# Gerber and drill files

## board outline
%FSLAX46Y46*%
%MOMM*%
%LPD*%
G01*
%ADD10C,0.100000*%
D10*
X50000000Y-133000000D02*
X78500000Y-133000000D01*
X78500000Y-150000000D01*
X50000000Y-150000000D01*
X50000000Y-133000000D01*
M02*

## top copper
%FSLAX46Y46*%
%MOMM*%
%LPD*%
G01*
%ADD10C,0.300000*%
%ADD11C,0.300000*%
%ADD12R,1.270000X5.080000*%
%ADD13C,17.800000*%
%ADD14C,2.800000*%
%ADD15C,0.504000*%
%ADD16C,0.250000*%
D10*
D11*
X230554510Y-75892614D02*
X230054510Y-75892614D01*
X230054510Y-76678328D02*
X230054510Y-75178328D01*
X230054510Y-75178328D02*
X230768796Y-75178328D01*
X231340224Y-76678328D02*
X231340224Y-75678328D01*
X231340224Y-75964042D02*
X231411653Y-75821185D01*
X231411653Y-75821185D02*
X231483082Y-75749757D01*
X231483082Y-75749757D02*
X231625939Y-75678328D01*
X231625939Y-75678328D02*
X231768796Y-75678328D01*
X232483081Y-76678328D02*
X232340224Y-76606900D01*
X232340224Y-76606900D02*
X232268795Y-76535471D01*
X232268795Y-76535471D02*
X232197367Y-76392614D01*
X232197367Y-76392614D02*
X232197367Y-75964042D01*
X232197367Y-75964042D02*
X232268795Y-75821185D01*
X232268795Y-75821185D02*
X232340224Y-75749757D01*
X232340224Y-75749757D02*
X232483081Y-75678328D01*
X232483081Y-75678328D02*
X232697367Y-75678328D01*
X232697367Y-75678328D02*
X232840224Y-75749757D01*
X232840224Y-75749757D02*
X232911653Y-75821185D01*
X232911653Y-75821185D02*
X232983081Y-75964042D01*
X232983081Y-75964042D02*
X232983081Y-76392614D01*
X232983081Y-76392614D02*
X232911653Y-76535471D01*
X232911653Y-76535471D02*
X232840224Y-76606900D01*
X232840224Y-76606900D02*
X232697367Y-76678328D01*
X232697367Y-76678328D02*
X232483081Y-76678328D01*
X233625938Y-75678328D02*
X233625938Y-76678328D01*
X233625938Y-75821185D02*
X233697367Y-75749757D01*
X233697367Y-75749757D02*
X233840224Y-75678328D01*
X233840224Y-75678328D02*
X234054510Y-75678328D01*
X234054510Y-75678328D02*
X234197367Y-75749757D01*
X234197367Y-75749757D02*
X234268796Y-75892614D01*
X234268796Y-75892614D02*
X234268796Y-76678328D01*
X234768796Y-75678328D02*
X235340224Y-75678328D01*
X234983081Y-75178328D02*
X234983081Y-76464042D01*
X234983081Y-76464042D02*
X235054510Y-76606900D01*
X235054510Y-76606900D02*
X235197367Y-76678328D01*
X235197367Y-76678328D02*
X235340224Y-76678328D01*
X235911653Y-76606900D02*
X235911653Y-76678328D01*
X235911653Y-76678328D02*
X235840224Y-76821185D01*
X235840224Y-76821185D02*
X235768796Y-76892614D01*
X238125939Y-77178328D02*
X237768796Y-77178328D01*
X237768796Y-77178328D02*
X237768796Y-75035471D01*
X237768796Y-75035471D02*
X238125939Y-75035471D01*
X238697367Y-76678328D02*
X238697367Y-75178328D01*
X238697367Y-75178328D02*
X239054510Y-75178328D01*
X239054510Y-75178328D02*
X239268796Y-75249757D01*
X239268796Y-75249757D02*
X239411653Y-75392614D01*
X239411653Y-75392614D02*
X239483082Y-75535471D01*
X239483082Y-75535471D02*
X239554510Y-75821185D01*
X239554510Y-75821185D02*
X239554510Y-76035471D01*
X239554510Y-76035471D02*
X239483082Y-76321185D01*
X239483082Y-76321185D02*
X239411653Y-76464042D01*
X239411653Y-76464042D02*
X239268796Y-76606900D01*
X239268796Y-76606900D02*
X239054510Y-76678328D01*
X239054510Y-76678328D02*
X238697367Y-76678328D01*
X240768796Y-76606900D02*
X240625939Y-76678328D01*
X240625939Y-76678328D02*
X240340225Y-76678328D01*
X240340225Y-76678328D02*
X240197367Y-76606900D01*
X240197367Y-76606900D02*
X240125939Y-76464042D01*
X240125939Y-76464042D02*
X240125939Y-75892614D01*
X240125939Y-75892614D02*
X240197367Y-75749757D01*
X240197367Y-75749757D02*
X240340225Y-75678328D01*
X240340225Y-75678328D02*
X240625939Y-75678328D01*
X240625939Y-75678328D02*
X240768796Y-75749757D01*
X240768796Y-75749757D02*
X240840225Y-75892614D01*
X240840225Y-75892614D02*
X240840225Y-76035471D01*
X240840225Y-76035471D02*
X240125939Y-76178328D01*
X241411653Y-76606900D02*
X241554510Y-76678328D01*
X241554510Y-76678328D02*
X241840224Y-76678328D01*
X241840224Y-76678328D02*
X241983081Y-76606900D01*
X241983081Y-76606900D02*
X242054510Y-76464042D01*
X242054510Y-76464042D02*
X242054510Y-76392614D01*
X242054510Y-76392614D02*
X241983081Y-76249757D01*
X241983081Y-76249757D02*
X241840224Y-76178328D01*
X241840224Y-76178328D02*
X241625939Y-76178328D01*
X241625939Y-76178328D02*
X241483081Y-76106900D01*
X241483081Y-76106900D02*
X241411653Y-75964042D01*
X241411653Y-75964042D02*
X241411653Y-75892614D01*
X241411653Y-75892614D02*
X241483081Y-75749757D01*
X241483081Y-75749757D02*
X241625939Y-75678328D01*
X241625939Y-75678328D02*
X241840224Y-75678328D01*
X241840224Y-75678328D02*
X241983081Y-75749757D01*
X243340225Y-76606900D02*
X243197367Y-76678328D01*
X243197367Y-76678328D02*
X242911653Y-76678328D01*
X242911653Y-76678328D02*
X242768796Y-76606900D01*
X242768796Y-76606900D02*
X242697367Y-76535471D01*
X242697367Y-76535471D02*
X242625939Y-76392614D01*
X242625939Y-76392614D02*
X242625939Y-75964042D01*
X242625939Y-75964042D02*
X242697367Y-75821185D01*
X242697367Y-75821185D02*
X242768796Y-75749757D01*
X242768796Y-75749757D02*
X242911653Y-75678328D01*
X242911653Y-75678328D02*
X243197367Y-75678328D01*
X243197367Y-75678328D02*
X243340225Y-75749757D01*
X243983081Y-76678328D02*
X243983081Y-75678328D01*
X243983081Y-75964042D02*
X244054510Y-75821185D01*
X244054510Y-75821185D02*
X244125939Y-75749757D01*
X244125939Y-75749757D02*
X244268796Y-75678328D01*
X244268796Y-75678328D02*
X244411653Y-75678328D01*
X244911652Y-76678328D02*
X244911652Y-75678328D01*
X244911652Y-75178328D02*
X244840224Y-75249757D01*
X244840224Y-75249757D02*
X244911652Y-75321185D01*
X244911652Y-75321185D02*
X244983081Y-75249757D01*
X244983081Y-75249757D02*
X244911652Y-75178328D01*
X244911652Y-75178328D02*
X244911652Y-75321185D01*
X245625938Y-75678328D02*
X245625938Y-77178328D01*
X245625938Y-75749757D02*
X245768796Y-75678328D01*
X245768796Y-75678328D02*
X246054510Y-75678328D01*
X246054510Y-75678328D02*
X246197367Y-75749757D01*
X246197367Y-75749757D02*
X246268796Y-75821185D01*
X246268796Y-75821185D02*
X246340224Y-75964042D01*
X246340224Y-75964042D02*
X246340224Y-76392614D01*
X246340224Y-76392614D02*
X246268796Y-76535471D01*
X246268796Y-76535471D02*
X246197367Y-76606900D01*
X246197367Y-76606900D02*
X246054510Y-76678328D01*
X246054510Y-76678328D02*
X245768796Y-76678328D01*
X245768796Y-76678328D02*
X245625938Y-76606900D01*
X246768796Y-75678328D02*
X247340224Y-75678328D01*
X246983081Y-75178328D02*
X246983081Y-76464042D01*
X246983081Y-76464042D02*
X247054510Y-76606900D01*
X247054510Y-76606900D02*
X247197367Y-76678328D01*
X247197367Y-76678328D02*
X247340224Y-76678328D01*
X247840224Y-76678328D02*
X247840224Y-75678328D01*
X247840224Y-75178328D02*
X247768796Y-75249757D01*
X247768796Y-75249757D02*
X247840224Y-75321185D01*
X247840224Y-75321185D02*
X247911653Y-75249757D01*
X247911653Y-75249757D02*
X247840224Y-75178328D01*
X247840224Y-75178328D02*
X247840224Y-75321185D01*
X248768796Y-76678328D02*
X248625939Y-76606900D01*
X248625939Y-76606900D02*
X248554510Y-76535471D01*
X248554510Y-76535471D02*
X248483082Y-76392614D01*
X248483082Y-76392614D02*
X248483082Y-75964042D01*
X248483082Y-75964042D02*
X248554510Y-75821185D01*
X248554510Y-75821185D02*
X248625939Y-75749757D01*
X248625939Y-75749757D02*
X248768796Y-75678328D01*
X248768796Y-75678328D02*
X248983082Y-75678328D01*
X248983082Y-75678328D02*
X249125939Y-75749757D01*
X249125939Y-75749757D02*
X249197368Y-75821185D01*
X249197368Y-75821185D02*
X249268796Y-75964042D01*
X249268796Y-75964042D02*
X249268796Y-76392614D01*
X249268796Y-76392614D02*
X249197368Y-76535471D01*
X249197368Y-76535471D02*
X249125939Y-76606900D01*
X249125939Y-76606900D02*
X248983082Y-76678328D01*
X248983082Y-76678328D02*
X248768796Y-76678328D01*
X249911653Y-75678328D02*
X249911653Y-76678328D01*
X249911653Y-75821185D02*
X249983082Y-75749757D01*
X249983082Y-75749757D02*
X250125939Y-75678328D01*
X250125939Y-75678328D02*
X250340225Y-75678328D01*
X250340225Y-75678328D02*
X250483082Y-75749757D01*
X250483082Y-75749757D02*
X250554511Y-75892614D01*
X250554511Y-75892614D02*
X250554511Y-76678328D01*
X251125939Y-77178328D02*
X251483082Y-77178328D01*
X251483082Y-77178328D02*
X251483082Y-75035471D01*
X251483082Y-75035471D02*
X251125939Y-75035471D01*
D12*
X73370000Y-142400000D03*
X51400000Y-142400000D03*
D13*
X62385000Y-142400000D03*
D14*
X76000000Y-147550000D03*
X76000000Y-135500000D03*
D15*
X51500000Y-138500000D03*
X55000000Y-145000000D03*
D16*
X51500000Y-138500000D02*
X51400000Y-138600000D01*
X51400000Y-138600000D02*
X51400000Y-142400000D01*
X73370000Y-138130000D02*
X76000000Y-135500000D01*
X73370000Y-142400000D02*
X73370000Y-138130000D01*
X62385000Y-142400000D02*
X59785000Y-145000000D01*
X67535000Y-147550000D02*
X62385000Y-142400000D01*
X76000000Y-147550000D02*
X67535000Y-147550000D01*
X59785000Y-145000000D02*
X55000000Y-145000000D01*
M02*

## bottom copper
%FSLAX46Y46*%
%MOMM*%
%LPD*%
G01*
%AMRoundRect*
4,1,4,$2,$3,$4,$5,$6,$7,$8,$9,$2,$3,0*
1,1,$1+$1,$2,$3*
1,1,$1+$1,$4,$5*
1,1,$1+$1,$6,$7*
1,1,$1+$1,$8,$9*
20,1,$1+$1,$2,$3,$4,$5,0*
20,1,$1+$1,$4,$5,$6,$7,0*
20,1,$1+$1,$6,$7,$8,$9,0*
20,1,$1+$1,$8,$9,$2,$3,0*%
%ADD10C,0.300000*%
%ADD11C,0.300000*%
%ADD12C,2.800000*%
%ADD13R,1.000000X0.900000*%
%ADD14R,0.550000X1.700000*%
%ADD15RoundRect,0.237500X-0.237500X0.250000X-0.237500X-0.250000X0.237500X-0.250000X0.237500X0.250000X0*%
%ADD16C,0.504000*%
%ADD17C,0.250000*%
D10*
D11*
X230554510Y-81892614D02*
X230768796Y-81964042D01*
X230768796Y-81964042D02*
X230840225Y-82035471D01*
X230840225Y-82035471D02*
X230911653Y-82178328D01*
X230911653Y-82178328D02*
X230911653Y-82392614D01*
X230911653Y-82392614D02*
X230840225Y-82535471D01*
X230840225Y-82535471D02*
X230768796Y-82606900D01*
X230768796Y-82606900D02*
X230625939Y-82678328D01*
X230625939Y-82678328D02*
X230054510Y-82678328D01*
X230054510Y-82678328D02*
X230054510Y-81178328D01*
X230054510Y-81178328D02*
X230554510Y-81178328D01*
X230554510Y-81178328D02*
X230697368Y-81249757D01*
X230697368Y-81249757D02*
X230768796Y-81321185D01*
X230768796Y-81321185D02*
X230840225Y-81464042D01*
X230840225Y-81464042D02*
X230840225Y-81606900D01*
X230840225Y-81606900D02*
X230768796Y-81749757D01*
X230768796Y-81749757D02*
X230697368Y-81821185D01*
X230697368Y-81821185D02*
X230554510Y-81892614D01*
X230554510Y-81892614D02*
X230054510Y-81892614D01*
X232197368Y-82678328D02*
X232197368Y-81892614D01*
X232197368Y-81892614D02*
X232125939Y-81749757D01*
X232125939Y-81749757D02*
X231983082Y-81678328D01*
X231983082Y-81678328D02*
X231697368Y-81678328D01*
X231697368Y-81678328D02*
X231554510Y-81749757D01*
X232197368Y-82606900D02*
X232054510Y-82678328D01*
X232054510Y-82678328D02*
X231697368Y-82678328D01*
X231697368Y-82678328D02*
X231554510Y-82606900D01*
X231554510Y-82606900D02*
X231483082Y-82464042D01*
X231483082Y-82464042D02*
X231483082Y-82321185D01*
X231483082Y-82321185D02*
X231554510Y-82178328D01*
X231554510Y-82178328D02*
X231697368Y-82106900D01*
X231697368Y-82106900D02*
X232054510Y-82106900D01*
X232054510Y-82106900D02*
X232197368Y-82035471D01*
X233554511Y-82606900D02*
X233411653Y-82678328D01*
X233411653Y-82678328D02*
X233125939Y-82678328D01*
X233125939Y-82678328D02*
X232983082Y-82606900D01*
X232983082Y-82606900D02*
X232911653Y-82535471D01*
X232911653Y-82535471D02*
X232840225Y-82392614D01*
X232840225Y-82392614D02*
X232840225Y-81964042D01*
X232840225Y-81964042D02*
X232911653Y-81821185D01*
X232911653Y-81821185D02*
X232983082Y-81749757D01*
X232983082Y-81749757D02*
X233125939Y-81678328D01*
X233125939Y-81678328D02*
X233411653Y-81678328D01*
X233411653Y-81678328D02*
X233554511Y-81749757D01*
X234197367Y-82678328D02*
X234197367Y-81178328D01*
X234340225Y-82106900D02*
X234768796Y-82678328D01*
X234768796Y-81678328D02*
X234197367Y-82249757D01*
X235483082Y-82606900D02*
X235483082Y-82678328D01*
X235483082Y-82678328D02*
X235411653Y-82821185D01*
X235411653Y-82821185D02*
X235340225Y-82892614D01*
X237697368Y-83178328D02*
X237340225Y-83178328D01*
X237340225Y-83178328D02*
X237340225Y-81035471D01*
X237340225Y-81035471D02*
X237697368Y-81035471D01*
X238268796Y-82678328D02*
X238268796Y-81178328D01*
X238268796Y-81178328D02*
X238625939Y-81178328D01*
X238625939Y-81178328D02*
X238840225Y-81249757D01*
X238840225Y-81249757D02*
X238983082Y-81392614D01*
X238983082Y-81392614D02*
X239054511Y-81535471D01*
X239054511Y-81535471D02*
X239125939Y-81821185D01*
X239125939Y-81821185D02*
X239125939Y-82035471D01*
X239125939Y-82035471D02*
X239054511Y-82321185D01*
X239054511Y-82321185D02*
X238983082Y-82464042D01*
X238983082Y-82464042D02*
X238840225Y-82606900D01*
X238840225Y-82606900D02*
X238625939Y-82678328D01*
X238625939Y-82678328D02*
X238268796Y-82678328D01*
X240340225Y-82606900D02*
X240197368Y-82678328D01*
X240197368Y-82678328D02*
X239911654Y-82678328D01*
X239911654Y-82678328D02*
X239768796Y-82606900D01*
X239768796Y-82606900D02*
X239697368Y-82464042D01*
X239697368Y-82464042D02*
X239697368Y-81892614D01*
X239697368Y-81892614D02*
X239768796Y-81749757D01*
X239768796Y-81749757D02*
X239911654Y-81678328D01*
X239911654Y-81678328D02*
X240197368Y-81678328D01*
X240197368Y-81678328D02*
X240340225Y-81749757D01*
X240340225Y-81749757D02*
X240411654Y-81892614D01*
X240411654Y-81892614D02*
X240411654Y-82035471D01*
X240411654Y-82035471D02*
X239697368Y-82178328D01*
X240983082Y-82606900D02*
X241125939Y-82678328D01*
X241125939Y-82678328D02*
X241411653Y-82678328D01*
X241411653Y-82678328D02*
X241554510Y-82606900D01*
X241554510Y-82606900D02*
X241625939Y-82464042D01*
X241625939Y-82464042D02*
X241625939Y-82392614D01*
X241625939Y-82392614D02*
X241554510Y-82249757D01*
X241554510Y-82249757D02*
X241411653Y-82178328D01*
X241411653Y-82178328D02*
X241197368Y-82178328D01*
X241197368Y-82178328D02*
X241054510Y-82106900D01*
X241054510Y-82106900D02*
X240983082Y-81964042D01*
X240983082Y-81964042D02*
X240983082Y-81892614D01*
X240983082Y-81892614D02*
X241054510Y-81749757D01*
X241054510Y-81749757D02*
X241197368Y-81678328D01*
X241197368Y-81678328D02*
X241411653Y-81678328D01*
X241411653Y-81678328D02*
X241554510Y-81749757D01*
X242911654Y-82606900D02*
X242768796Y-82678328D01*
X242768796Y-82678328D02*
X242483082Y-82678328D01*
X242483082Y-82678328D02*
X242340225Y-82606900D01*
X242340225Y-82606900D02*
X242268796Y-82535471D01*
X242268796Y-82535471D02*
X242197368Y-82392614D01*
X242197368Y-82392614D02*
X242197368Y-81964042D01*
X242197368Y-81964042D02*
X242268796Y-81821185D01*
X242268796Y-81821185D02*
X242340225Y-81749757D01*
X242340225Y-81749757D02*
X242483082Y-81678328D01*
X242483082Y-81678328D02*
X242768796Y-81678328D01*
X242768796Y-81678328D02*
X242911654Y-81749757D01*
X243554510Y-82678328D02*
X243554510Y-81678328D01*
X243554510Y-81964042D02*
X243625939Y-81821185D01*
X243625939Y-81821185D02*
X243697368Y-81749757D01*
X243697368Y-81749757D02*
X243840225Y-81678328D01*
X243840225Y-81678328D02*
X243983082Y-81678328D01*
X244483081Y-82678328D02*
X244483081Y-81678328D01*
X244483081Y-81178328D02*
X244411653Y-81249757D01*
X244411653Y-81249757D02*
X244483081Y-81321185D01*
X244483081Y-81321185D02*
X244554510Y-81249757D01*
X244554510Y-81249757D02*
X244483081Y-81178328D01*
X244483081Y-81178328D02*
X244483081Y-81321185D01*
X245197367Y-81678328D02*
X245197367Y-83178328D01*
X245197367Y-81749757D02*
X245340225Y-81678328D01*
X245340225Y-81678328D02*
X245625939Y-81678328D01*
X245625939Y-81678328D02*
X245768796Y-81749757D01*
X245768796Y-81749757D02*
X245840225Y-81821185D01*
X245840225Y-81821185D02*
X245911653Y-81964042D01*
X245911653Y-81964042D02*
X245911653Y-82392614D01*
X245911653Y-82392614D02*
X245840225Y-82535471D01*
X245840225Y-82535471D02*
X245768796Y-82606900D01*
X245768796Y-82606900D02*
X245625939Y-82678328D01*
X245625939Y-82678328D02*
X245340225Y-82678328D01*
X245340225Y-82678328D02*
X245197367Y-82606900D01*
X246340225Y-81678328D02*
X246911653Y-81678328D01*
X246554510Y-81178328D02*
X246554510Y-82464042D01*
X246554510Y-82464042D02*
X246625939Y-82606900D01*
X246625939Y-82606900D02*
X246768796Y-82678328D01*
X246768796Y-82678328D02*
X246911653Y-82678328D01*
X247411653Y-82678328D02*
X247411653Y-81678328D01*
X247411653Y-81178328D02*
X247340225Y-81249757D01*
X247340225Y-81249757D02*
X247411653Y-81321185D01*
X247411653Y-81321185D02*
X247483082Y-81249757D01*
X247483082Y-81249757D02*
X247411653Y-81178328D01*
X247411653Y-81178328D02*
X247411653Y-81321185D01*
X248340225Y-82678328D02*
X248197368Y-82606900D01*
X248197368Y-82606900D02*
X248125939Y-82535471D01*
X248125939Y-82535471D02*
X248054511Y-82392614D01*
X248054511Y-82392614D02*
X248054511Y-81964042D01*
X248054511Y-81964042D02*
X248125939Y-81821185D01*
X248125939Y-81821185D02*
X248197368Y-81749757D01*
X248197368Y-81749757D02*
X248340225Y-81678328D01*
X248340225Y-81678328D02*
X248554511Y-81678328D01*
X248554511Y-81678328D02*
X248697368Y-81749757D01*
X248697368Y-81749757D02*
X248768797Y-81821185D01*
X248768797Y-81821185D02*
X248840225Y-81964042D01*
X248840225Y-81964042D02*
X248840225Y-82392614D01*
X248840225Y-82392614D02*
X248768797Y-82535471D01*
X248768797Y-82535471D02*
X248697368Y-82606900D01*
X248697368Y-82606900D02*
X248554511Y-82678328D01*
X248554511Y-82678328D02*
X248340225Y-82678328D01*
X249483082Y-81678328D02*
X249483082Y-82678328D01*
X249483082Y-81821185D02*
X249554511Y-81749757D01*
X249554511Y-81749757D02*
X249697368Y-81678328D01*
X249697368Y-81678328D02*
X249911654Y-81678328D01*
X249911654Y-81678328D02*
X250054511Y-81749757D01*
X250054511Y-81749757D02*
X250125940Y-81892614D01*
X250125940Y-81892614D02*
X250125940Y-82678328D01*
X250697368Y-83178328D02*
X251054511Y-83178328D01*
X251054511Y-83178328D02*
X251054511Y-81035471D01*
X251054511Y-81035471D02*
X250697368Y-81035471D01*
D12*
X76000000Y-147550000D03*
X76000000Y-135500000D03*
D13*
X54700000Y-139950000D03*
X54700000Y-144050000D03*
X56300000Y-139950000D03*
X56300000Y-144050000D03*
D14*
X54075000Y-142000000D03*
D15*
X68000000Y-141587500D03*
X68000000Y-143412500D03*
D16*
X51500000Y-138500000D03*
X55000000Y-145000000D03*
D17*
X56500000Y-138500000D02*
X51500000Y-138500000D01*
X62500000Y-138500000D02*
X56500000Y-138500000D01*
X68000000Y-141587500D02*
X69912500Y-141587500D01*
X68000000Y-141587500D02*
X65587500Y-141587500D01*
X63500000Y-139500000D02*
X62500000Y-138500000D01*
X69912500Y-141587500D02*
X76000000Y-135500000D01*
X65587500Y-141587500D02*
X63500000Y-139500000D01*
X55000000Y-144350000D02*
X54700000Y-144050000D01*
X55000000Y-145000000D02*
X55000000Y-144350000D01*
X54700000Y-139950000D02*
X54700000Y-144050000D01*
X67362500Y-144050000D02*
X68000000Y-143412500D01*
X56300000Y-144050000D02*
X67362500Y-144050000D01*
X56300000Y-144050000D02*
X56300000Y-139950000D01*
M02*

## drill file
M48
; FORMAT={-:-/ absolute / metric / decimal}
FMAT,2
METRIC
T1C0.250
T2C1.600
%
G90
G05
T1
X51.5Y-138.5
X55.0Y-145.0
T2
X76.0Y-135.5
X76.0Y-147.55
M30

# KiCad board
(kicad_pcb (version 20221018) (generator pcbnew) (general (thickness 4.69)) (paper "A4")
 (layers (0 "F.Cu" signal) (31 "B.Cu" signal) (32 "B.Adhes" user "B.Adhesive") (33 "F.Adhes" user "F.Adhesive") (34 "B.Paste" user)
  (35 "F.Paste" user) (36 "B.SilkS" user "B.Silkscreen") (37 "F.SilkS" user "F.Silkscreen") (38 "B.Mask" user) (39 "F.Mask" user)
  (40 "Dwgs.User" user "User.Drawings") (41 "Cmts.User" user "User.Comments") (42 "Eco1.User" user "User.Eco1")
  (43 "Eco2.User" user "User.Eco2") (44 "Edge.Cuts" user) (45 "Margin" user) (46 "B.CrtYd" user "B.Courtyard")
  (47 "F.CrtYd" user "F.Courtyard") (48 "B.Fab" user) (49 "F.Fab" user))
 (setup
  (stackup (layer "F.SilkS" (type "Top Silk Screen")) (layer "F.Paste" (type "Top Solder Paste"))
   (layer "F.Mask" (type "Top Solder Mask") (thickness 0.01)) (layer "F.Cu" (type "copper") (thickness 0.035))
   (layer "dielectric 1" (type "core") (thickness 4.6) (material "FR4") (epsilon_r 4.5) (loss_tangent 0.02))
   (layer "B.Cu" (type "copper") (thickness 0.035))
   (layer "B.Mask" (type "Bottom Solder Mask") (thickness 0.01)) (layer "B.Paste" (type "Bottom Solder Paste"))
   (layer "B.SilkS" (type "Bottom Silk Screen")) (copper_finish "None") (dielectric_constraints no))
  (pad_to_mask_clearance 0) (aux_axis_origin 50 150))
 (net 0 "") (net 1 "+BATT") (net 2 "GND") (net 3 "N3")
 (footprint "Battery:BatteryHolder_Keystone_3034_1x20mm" (layer "F.Cu") (at 62.385 142.4 180)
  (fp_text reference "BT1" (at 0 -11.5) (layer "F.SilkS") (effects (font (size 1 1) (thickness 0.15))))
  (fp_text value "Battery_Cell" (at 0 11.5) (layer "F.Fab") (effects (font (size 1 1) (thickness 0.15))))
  (pad "1" smd rect (at -10.985 0 180) (size 1.27 5.08) (layers "F.Cu" "F.Paste" "F.Mask") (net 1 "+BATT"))
  (pad "1" smd rect (at 10.985 0 180) (size 1.27 5.08) (layers "F.Cu" "F.Paste" "F.Mask") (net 1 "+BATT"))
  (pad "2" smd circle (at 0 0 180) (size 17.8 17.8) (layers "F.Cu" "F.Mask") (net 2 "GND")))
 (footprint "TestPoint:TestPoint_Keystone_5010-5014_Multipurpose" (layer "F.Cu") (at 76 147.55)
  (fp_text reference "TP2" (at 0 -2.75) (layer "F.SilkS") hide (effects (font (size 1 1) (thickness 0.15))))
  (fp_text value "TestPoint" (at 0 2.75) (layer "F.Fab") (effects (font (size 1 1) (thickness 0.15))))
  (pad "1" thru_hole circle (at 0 0) (size 2.8 2.8) (drill 1.6) (layers "*.Cu" "*.Mask") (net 2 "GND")))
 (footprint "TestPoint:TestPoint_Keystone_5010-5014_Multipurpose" (layer "F.Cu") (at 76 135.5)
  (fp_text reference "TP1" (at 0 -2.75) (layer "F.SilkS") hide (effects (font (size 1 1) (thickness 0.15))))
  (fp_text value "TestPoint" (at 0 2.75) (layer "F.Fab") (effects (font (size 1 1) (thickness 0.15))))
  (pad "1" thru_hole circle (at 0 0) (size 2.8 2.8) (drill 1.6) (layers "*.Cu" "*.Mask") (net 1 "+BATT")))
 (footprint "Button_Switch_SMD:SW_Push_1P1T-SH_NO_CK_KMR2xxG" (layer "B.Cu") (at 55.5 142 -90)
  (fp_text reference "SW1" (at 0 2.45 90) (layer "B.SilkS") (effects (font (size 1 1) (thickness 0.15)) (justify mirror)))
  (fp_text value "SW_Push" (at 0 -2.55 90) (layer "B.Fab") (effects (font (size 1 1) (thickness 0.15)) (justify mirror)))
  (pad "1" smd rect (at -2.05 0.8 270) (size 0.9 1) (layers "B.Cu" "B.Paste" "B.Mask") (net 2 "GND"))
  (pad "1" smd rect (at 2.05 0.8 270) (size 0.9 1) (layers "B.Cu" "B.Paste" "B.Mask") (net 2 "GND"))
  (pad "2" smd rect (at -2.05 -0.8 270) (size 0.9 1) (layers "B.Cu" "B.Paste" "B.Mask") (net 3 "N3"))
  (pad "2" smd rect (at 2.05 -0.8 270) (size 0.9 1) (layers "B.Cu" "B.Paste" "B.Mask") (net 3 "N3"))
  (pad "SH" smd rect (at 0 1.425 270) (size 1.7 0.55) (layers "B.Cu" "B.Paste" "B.Mask")))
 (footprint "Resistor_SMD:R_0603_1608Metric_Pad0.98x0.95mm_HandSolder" (layer "B.Cu") (at 68 142.5 -90)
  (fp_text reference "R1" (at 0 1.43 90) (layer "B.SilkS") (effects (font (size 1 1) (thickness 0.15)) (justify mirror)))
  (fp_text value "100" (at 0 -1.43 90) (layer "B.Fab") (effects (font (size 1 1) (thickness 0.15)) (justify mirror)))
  (pad "1" smd roundrect (at -0.9125 0 270) (size 0.975 0.95) (layers "B.Cu" "B.Paste" "B.Mask") (roundrect_rratio 0.25) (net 1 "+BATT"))
  (pad "2" smd roundrect (at 0.9125 0 270) (size 0.975 0.95) (layers "B.Cu" "B.Paste" "B.Mask") (roundrect_rratio 0.25) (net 3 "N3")))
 (gr_rect (start 50 133) (end 78.5 150) (stroke (width 0.1) (type default)) (fill none) (layer "Edge.Cuts"))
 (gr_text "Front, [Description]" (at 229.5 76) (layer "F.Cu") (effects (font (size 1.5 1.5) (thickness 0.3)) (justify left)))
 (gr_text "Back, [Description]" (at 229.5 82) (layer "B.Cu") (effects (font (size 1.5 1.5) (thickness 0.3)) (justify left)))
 (segment (start 51.5 138.5) (end 51.4 138.6) (width 0.25) (layer "F.Cu") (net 1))
 (segment (start 51.4 138.6) (end 51.4 142.4) (width 0.25) (layer "F.Cu") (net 1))
 (segment (start 73.37 138.13) (end 76 135.5) (width 0.25) (layer "F.Cu") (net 1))
 (segment (start 73.37 142.4) (end 73.37 138.13) (width 0.25) (layer "F.Cu") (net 1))
 (via (at 51.5 138.5) (size 0.504) (drill 0.25) (layers "F.Cu" "B.Cu") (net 1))
 (segment (start 56.5 138.5) (end 51.5 138.5) (width 0.25) (layer "B.Cu") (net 1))
 (segment (start 62.5 138.5) (end 56.5 138.5) (width 0.25) (layer "B.Cu") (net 1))
 (segment (start 68 141.5875) (end 69.9125 141.5875) (width 0.25) (layer "B.Cu") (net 1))
 (segment (start 68 141.5875) (end 65.5875 141.5875) (width 0.25) (layer "B.Cu") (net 1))
 (segment (start 63.5 139.5) (end 62.5 138.5) (width 0.25) (layer "B.Cu") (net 1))
 (segment (start 69.9125 141.5875) (end 76 135.5) (width 0.25) (layer "B.Cu") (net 1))
 (segment (start 65.5875 141.5875) (end 63.5 139.5) (width 0.25) (layer "B.Cu") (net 1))
 (segment (start 62.385 142.4) (end 59.785 145) (width 0.25) (layer "F.Cu") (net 2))
 (segment (start 67.535 147.55) (end 62.385 142.4) (width 0.25) (layer "F.Cu") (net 2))
 (segment (start 76 147.55) (end 67.535 147.55) (width 0.25) (layer "F.Cu") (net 2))
 (segment (start 59.785 145) (end 55 145) (width 0.25) (layer "F.Cu") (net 2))
 (via (at 55 145) (size 0.504) (drill 0.25) (layers "F.Cu" "B.Cu") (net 2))
 (segment (start 55 144.35) (end 54.7 144.05) (width 0.25) (layer "B.Cu") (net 2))
 (segment (start 55 145) (end 55 144.35) (width 0.25) (layer "B.Cu") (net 2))
 (segment (start 54.7 139.95) (end 54.7 144.05) (width 0.25) (layer "B.Cu") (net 2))
 (segment (start 67.3625 144.05) (end 68 143.4125) (width 0.25) (layer "B.Cu") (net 3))
 (segment (start 56.3 144.05) (end 67.3625 144.05) (width 0.25) (layer "B.Cu") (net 3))
 (segment (start 56.3 144.05) (end 56.3 139.95) (width 0.25) (layer "B.Cu") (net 3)))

